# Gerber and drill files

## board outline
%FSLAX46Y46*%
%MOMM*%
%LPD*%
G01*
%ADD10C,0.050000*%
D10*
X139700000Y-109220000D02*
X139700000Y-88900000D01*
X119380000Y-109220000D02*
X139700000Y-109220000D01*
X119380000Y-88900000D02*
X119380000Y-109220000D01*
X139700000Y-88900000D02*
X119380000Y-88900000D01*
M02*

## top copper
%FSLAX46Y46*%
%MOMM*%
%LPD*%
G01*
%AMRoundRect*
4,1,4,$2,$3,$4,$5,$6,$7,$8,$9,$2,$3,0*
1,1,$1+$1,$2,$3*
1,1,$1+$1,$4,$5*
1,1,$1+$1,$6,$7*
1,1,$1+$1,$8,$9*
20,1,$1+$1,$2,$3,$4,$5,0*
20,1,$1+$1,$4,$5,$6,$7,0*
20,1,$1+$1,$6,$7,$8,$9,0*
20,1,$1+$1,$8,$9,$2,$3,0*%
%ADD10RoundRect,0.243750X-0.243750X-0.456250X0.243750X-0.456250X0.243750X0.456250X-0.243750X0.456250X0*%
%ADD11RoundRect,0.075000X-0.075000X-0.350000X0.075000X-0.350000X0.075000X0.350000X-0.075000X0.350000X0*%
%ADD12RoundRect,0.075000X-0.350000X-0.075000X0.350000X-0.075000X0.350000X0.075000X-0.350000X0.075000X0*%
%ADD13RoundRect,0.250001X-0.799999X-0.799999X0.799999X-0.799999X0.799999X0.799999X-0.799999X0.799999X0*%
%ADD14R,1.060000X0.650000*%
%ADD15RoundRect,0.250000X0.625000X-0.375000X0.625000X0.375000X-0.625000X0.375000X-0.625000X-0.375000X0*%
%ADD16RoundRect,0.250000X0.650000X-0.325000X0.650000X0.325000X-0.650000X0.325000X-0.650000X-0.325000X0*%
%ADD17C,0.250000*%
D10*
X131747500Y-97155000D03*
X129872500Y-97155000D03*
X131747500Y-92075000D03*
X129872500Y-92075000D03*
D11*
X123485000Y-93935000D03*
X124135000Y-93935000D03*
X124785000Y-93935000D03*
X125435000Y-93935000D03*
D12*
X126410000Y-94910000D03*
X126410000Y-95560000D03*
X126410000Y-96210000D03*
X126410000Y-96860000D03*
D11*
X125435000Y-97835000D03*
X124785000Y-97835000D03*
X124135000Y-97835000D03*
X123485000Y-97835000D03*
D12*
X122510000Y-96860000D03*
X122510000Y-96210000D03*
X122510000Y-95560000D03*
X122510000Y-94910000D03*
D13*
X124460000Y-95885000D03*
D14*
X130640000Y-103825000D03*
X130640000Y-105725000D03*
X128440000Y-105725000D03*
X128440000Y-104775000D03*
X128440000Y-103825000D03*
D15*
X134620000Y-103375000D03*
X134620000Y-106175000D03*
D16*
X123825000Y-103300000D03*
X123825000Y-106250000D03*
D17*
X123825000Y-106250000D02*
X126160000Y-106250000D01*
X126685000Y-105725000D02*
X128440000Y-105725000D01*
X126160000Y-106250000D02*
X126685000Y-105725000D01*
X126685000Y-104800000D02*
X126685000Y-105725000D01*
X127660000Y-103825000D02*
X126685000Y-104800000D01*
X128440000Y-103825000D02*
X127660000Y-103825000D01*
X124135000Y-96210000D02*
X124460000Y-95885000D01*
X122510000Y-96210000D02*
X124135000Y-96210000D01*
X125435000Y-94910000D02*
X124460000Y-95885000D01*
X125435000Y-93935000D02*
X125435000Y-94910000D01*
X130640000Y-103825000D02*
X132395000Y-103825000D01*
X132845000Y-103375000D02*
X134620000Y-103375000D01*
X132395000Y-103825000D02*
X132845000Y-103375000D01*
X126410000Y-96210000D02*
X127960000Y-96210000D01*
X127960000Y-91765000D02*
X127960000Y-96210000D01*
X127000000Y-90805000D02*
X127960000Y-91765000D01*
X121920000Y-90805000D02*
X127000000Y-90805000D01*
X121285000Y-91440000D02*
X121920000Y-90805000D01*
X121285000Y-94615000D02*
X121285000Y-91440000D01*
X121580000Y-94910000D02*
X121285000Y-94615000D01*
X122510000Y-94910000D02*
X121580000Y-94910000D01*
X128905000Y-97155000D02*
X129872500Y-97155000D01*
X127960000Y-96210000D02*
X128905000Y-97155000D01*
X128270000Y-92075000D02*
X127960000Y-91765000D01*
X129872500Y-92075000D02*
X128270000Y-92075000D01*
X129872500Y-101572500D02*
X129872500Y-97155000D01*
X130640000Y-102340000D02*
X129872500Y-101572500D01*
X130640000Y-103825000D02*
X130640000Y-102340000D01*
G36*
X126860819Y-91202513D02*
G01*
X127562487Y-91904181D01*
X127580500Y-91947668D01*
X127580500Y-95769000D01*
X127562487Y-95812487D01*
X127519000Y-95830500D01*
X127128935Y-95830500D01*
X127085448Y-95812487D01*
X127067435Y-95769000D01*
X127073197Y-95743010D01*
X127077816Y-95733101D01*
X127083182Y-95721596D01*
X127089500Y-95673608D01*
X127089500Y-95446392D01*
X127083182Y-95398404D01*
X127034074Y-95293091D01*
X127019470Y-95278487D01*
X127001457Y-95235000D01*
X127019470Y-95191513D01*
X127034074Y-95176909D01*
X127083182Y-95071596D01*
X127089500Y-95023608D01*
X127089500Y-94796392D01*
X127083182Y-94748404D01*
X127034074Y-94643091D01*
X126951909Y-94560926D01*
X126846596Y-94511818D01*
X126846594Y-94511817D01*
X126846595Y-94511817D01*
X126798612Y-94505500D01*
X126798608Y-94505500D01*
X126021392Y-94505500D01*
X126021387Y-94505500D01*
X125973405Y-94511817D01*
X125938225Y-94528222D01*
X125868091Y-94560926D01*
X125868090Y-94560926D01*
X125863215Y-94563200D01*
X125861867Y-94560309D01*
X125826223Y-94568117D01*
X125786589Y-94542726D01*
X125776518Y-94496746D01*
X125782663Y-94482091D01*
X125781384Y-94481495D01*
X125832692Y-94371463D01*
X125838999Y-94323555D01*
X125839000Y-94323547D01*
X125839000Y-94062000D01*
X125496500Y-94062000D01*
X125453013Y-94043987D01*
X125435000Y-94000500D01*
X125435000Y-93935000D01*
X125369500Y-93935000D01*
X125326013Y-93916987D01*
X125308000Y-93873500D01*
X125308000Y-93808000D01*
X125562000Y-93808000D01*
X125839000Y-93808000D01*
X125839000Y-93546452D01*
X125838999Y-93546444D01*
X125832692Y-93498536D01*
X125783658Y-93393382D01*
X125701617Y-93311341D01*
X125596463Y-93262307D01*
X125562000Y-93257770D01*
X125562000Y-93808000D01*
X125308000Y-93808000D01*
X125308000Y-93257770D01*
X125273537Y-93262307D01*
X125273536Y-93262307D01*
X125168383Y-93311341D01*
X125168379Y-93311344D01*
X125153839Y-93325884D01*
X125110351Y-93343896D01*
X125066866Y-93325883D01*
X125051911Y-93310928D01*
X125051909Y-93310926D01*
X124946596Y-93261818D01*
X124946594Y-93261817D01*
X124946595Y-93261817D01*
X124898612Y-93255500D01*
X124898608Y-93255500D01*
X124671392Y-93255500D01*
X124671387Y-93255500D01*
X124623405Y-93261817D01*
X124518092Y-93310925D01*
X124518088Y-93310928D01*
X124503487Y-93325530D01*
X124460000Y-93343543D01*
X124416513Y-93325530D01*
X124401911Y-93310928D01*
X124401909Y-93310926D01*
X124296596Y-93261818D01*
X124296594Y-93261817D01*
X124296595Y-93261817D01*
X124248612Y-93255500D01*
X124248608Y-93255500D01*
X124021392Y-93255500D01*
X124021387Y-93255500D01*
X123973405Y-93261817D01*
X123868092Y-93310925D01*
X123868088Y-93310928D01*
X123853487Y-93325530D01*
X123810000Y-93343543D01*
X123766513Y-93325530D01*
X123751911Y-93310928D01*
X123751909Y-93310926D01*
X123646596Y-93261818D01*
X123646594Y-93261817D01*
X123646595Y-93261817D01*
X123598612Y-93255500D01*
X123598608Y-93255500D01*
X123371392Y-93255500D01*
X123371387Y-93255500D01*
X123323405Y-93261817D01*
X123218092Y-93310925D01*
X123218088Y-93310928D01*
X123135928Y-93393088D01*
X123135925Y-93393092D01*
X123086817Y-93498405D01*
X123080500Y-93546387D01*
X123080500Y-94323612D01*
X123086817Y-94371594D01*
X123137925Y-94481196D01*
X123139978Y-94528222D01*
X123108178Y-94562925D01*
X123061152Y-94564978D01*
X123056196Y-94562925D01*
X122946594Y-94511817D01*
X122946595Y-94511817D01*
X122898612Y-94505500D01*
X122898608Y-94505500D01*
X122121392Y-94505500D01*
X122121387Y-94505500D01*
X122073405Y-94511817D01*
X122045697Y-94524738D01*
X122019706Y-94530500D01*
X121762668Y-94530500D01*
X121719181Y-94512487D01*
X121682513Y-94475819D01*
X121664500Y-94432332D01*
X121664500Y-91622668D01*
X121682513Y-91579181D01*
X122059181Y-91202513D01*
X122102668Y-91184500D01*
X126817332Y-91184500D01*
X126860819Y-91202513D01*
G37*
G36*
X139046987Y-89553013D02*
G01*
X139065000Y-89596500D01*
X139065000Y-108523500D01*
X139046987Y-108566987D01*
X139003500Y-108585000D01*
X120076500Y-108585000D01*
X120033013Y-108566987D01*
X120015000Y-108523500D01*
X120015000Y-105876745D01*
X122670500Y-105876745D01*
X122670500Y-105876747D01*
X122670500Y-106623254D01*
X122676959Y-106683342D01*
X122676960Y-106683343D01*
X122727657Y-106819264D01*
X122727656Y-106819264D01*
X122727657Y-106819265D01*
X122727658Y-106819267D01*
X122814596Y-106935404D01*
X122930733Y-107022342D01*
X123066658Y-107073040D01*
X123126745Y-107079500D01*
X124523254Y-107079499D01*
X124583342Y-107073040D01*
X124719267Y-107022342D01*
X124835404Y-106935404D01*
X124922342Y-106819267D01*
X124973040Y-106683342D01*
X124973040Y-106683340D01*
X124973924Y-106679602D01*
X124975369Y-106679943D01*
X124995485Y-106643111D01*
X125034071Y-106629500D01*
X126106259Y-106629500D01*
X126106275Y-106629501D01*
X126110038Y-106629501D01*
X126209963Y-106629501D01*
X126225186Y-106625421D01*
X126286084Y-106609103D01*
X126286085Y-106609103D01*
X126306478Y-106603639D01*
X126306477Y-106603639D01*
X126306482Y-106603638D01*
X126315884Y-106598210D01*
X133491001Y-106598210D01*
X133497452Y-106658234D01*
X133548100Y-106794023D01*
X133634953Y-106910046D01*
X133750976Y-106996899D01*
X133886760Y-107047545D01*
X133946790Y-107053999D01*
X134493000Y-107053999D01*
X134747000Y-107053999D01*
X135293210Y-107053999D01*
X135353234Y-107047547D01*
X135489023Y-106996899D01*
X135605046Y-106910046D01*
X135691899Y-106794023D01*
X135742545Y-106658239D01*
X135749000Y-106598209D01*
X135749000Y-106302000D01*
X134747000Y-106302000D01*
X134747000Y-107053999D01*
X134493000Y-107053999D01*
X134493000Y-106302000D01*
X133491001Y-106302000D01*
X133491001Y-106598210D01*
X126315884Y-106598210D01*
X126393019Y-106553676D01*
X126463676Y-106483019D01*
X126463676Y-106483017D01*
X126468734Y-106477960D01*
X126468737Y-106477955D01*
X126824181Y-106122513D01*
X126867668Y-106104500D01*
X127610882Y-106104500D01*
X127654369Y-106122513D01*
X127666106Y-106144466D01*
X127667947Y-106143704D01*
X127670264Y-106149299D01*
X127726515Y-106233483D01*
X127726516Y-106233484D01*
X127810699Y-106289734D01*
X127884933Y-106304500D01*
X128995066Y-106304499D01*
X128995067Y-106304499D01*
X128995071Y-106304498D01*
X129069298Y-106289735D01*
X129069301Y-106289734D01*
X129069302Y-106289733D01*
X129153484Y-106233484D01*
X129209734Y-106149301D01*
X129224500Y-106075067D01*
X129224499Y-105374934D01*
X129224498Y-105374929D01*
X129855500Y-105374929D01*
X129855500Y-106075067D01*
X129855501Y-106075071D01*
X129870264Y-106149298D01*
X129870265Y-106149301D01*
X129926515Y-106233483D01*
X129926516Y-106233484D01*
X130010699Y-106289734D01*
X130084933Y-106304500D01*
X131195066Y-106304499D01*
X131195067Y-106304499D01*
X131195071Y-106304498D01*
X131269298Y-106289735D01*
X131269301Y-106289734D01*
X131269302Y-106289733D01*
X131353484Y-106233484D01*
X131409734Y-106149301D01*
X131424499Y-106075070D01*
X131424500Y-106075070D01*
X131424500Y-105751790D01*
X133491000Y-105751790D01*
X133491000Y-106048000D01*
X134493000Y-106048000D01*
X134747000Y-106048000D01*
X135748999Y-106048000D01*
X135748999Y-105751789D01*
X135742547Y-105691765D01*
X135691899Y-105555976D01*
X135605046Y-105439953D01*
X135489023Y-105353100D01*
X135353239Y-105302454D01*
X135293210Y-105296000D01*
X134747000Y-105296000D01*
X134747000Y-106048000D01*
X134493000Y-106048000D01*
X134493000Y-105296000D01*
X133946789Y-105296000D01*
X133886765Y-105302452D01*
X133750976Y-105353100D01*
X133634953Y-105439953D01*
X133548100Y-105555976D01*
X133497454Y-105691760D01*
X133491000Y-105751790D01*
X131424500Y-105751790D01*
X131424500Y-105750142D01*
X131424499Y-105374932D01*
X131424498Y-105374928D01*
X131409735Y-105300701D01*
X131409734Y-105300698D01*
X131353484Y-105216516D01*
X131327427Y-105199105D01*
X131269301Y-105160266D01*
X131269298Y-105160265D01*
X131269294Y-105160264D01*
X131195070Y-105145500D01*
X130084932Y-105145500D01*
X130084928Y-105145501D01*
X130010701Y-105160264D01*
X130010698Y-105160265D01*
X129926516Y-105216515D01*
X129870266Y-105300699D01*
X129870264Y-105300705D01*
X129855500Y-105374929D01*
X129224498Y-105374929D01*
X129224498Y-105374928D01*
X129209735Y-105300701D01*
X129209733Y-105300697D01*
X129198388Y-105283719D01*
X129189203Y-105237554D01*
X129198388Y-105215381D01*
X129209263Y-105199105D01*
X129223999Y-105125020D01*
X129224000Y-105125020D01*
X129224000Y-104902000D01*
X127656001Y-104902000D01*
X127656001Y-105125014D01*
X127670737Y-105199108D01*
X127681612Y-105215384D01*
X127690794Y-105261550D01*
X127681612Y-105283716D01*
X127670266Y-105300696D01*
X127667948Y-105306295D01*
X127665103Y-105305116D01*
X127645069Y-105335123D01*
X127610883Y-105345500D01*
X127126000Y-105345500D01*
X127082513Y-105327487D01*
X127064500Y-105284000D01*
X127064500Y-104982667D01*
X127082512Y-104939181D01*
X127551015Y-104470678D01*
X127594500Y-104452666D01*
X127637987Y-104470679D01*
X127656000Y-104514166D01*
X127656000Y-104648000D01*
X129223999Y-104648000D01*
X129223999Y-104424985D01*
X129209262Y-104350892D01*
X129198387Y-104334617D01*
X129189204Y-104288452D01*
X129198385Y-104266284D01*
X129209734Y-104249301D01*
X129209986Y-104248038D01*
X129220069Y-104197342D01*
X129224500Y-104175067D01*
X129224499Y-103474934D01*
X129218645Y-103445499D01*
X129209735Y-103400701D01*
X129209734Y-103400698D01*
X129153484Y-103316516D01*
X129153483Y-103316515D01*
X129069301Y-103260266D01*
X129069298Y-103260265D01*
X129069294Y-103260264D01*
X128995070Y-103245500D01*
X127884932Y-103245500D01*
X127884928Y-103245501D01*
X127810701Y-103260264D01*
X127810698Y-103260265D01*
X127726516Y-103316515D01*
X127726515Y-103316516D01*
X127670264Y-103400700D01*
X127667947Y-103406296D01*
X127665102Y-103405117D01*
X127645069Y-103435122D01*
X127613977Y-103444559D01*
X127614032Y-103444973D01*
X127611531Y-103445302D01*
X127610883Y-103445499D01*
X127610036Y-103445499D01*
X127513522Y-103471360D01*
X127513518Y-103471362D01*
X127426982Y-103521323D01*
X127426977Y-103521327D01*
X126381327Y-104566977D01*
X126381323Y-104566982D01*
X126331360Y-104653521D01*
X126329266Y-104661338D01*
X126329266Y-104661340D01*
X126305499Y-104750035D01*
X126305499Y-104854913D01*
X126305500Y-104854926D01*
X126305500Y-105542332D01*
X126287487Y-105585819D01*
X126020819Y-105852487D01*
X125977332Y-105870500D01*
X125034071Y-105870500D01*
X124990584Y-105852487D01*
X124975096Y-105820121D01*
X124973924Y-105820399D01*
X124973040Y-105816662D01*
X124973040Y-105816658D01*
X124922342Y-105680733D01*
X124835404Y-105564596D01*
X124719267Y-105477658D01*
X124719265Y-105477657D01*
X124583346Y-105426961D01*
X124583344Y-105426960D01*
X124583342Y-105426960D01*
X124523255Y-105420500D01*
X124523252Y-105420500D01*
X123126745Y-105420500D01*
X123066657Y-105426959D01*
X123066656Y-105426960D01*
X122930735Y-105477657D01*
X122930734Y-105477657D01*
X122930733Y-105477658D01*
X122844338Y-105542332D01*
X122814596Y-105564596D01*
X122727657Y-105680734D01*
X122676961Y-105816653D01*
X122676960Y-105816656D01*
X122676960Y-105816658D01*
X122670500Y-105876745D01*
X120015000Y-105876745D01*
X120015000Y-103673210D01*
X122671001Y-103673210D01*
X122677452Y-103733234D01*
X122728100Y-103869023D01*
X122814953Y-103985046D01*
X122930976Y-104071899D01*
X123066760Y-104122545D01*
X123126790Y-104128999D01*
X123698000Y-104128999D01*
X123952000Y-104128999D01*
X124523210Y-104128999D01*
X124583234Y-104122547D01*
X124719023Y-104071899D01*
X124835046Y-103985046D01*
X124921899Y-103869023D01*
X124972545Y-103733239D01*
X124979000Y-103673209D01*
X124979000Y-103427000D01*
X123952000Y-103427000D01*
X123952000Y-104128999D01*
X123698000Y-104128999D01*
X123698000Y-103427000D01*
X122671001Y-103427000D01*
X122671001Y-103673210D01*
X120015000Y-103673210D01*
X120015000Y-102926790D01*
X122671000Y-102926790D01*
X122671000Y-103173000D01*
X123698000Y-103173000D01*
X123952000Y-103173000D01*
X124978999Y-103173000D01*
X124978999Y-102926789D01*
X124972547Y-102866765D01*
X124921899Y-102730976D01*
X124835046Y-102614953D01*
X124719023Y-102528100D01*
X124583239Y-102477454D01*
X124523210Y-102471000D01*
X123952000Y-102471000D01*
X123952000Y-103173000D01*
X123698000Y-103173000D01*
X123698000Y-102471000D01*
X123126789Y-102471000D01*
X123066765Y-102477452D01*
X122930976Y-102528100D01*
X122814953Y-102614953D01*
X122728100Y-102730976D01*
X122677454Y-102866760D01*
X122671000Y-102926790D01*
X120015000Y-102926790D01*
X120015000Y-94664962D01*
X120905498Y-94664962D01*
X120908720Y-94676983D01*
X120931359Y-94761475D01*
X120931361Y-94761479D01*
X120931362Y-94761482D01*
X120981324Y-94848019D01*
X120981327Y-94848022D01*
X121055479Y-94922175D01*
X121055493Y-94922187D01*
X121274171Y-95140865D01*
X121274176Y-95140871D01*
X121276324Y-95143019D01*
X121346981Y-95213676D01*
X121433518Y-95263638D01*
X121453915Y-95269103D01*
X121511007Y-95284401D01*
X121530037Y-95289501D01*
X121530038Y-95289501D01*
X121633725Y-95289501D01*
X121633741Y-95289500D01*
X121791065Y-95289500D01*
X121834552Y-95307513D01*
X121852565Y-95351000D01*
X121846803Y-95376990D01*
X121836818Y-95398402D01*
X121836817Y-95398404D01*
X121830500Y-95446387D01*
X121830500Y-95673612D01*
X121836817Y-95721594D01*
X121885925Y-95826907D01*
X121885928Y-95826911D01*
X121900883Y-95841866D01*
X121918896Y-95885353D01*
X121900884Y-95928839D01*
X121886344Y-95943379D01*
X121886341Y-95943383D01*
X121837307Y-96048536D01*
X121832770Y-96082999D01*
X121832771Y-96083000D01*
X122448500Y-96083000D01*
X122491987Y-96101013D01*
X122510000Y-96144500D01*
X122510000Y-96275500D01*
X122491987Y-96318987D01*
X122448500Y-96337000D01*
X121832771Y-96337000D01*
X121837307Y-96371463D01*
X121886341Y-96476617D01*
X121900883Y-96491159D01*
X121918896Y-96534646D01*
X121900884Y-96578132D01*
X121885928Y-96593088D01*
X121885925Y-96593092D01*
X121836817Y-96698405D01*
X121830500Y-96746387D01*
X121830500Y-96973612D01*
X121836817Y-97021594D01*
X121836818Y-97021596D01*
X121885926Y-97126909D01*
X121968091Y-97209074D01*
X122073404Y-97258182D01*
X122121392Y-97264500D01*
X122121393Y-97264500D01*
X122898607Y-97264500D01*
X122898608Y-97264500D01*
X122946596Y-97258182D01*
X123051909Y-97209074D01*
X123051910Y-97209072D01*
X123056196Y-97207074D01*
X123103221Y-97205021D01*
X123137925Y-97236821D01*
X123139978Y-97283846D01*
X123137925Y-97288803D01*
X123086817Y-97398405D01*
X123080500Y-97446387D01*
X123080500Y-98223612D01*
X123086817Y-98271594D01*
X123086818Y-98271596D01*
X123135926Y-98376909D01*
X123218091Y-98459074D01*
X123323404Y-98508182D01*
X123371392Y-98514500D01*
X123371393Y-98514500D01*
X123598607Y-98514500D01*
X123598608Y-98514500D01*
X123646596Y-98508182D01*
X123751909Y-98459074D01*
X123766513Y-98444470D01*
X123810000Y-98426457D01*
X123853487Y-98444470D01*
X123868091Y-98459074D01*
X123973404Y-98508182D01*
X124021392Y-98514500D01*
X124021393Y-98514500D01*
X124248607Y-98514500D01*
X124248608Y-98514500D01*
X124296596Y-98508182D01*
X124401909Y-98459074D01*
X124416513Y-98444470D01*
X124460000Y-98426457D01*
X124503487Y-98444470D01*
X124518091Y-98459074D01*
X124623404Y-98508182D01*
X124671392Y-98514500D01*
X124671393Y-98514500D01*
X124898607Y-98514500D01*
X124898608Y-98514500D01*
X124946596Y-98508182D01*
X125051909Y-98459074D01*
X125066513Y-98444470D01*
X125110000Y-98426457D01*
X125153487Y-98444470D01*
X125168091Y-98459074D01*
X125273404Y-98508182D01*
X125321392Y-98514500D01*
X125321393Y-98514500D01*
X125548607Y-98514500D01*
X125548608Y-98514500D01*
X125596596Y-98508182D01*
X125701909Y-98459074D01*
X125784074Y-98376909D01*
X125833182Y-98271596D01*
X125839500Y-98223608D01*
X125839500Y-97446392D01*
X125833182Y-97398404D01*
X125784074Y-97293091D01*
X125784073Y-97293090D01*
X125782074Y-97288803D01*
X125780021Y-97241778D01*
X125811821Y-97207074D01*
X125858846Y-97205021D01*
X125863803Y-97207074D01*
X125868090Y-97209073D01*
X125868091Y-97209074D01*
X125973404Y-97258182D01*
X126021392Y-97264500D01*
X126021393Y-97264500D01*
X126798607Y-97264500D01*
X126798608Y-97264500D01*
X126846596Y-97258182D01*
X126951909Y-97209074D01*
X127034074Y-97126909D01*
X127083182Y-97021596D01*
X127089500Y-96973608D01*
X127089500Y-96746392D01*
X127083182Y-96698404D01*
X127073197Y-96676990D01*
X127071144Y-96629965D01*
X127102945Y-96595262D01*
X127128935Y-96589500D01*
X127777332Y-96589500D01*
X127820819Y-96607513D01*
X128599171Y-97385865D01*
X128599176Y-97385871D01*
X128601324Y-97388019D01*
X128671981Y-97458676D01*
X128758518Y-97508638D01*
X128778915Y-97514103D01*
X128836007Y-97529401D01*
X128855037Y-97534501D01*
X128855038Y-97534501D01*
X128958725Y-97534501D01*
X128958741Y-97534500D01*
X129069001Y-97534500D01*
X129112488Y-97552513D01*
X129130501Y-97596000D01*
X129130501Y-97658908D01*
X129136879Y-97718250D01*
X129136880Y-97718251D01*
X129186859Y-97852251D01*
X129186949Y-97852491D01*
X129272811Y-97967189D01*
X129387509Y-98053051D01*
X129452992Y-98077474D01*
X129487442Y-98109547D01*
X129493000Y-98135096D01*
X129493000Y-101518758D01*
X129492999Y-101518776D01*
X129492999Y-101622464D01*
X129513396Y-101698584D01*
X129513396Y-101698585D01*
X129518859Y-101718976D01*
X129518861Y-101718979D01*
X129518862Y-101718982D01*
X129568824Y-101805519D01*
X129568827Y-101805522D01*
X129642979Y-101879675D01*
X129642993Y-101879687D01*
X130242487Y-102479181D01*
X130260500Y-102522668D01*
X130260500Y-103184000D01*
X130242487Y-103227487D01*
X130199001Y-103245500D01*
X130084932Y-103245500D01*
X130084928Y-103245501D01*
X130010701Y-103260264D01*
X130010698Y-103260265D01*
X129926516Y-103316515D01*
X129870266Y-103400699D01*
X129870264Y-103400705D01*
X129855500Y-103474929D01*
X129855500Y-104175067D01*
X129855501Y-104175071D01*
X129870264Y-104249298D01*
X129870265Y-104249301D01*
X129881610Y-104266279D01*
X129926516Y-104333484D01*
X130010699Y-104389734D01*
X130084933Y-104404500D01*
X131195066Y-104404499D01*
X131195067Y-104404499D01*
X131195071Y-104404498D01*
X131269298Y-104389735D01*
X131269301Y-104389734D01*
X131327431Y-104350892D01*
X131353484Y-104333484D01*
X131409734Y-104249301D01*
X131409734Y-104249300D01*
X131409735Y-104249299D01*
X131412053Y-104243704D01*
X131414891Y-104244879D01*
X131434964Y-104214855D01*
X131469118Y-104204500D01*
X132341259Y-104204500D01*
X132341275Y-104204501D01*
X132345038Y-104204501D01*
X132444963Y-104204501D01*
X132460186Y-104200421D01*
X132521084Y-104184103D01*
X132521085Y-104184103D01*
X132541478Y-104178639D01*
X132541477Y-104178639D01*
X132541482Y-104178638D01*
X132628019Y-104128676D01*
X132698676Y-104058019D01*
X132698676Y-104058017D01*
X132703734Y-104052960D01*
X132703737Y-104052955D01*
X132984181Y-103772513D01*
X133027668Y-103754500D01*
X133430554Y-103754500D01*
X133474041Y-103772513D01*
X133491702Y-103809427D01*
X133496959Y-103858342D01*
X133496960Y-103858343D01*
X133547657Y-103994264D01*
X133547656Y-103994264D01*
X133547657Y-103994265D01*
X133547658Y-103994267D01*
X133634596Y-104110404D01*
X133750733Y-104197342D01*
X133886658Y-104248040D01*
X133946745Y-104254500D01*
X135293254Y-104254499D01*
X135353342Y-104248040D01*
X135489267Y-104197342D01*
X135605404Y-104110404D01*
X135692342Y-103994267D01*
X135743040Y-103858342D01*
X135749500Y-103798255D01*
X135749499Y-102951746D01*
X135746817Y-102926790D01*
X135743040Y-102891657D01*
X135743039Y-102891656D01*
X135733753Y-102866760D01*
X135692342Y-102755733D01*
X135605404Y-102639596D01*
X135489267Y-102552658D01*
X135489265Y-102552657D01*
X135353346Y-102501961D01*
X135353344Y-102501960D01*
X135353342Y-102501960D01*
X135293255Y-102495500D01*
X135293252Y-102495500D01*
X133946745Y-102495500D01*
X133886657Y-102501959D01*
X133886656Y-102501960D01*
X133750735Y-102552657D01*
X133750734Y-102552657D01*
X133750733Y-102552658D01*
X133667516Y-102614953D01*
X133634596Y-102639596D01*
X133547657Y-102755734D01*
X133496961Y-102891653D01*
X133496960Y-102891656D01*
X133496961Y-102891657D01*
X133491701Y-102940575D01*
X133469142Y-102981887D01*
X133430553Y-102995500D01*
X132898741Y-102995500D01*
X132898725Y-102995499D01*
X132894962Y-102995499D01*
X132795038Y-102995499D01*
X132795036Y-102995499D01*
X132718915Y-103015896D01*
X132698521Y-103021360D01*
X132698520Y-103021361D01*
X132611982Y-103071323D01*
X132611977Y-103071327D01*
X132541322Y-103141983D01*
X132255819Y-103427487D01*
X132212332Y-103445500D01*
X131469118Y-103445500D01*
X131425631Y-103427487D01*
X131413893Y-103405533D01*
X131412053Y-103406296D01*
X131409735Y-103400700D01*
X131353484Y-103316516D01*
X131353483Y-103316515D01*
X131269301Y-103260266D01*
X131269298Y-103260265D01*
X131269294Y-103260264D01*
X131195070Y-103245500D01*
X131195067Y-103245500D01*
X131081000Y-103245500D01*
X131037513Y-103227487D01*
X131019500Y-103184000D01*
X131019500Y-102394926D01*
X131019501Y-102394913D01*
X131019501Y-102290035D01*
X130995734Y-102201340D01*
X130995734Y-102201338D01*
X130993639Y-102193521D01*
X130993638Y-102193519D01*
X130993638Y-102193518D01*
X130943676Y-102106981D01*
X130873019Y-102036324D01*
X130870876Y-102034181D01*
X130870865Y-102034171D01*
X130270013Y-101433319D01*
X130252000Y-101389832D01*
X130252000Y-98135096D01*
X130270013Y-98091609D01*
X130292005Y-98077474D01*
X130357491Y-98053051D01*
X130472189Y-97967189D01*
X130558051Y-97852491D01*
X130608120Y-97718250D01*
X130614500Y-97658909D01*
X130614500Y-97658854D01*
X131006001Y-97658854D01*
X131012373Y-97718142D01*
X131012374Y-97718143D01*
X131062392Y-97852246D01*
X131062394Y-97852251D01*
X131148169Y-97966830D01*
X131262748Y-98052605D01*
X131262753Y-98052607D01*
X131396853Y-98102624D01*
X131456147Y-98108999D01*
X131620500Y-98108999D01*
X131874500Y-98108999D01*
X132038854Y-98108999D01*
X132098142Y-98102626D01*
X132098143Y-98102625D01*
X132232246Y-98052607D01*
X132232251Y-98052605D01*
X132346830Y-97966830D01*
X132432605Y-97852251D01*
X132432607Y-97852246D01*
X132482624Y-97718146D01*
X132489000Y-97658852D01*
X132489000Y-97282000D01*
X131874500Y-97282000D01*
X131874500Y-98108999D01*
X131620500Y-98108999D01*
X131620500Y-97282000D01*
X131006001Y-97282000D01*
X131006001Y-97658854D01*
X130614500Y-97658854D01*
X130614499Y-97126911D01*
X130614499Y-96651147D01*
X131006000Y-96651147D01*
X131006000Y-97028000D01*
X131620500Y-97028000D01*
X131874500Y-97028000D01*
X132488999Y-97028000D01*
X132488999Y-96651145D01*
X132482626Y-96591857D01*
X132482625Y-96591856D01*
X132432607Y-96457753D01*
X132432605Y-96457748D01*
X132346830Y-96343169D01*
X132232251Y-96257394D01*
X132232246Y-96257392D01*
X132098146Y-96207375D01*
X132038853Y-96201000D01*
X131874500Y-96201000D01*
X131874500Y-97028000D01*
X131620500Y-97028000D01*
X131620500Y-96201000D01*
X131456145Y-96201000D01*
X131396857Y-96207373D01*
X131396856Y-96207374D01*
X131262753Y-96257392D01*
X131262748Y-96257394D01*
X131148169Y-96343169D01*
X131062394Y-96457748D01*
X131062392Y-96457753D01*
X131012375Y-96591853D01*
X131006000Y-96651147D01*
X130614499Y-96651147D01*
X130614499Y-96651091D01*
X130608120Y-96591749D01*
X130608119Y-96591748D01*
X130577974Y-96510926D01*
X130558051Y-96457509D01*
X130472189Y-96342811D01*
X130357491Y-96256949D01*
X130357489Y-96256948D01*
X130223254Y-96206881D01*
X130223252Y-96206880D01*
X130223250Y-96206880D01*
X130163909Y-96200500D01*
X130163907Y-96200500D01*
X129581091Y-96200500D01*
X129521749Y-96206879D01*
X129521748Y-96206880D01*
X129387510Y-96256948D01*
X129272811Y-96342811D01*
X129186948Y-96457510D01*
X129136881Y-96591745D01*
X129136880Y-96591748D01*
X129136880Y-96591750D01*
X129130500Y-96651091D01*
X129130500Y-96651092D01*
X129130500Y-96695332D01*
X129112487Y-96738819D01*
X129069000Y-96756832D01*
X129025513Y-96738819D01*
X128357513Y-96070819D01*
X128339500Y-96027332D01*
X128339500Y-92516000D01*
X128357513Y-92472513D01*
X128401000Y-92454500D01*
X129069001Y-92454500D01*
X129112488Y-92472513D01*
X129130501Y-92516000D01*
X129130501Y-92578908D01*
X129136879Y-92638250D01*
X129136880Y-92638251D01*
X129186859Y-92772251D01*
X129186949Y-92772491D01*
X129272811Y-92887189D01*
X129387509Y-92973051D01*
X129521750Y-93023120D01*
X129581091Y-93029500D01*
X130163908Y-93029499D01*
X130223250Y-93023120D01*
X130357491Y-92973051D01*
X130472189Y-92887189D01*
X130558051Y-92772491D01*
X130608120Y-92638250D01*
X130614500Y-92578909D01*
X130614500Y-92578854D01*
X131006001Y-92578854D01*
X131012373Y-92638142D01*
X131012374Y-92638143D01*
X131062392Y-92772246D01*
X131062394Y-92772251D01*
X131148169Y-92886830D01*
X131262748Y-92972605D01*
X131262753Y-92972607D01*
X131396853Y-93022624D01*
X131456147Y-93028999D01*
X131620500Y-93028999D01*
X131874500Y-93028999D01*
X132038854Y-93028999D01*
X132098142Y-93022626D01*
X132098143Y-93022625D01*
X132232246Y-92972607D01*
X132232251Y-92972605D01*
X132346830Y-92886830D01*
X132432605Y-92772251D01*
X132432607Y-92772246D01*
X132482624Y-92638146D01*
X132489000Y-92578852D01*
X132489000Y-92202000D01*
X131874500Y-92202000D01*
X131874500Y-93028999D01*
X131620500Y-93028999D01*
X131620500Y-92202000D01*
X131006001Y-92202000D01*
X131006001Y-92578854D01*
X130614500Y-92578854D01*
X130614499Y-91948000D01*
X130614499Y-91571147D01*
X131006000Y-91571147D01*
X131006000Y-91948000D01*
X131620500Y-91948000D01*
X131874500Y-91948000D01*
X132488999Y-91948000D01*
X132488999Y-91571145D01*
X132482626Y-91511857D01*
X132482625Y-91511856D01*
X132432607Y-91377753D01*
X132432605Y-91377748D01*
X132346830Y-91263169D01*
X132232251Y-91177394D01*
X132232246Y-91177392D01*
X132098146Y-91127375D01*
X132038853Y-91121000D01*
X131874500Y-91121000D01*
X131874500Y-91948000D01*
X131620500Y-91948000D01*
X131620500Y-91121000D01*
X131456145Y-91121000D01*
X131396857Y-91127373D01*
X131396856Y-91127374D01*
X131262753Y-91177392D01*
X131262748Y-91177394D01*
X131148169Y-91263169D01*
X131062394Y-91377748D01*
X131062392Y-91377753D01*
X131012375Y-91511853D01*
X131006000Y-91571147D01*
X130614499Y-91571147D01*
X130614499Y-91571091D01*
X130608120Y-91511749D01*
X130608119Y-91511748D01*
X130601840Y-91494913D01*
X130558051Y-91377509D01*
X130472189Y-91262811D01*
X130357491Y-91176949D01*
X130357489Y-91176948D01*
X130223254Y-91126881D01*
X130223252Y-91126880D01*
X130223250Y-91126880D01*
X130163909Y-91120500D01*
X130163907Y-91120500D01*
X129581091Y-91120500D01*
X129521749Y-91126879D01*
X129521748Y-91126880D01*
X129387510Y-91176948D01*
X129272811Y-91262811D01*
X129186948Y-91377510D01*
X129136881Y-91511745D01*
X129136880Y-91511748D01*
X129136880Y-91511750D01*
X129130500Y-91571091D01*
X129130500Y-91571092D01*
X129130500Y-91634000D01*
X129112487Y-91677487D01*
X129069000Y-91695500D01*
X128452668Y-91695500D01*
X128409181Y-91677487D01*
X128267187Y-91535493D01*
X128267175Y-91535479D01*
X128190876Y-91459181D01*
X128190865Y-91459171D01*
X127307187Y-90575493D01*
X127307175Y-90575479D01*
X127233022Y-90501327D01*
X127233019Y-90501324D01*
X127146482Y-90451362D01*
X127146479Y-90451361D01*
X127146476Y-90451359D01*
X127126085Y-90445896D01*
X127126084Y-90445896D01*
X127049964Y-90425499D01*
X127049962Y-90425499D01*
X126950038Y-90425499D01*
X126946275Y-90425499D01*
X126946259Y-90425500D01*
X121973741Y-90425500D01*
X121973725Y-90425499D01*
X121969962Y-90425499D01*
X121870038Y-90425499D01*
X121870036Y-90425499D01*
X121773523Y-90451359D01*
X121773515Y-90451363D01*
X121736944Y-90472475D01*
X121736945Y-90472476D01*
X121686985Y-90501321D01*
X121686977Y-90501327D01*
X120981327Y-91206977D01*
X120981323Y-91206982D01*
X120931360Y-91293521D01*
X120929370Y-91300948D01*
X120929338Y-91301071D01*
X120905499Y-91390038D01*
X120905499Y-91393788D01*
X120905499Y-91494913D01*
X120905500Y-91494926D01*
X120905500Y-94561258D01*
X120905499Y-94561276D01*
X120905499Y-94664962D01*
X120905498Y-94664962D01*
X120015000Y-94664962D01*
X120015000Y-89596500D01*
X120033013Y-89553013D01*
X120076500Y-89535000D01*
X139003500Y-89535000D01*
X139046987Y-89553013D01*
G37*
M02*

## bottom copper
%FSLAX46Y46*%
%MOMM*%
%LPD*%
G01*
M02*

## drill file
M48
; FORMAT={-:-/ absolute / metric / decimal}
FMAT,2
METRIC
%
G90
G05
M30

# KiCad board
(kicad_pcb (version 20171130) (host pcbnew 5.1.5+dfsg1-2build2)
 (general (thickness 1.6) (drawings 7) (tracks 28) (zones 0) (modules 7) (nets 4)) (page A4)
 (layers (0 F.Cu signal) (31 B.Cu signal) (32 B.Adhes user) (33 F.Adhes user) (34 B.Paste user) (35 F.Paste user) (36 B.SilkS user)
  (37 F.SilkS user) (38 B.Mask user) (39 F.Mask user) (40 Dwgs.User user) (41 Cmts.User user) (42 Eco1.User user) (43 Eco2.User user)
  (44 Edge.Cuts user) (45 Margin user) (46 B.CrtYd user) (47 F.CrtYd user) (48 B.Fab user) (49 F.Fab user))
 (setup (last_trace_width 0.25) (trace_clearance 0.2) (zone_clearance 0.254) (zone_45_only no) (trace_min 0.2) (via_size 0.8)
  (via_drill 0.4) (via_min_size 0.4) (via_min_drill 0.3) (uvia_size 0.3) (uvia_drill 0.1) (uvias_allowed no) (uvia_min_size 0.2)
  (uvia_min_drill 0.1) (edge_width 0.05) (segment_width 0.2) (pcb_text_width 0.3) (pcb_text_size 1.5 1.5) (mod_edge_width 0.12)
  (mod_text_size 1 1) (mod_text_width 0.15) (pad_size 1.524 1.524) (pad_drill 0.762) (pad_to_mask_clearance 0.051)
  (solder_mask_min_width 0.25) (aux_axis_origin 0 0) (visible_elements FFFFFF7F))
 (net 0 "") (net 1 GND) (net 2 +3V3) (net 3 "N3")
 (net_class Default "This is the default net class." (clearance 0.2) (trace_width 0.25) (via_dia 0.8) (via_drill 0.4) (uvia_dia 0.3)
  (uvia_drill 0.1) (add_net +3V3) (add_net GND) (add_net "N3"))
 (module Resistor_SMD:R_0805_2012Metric (layer F.Cu) (at 130.81 97.155)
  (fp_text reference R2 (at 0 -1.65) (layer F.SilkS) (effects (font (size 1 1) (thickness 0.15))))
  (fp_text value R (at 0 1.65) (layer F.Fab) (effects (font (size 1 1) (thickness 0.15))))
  (pad 2 smd roundrect (at 0.9375 0) (size 0.975 1.4) (layers F.Cu F.Paste F.Mask) (roundrect_rratio 0.25) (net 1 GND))
  (pad 1 smd roundrect (at -0.9375 0) (size 0.975 1.4) (layers F.Cu F.Paste F.Mask) (roundrect_rratio 0.25) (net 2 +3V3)))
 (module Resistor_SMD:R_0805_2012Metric (layer F.Cu) (at 130.81 92.075)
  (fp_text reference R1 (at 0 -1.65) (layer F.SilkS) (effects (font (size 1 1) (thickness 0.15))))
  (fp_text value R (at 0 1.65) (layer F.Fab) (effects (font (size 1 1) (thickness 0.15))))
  (pad 2 smd roundrect (at 0.9375 0) (size 0.975 1.4) (layers F.Cu F.Paste F.Mask) (roundrect_rratio 0.25) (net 1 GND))
  (pad 1 smd roundrect (at -0.9375 0) (size 0.975 1.4) (layers F.Cu F.Paste F.Mask) (roundrect_rratio 0.25) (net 2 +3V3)))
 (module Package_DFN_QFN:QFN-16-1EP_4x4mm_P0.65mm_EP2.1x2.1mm (layer F.Cu) (at 124.46 95.885)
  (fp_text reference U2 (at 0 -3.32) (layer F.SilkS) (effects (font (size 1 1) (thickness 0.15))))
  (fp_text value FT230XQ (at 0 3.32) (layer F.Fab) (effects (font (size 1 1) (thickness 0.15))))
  (pad 16 smd roundrect (at -0.975 -1.95) (size 0.3 0.85) (layers F.Cu F.Paste F.Mask) (roundrect_rratio 0.25))
  (pad 15 smd roundrect (at -0.325 -1.95) (size 0.3 0.85) (layers F.Cu F.Paste F.Mask) (roundrect_rratio 0.25))
  (pad 14 smd roundrect (at 0.325 -1.95) (size 0.3 0.85) (layers F.Cu F.Paste F.Mask) (roundrect_rratio 0.25))
  (pad 13 smd roundrect (at 0.975 -1.95) (size 0.3 0.85) (layers F.Cu F.Paste F.Mask) (roundrect_rratio 0.25) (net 1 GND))
  (pad 12 smd roundrect (at 1.95 -0.975) (size 0.85 0.3) (layers F.Cu F.Paste F.Mask) (roundrect_rratio 0.25))
  (pad 11 smd roundrect (at 1.95 -0.325) (size 0.85 0.3) (layers F.Cu F.Paste F.Mask) (roundrect_rratio 0.25))
  (pad 10 smd roundrect (at 1.95 0.325) (size 0.85 0.3) (layers F.Cu F.Paste F.Mask) (roundrect_rratio 0.25) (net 2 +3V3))
  (pad 9 smd roundrect (at 1.95 0.975) (size 0.85 0.3) (layers F.Cu F.Paste F.Mask) (roundrect_rratio 0.25))
  (pad 8 smd roundrect (at 0.975 1.95) (size 0.3 0.85) (layers F.Cu F.Paste F.Mask) (roundrect_rratio 0.25))
  (pad 7 smd roundrect (at 0.325 1.95) (size 0.3 0.85) (layers F.Cu F.Paste F.Mask) (roundrect_rratio 0.25))
  (pad 6 smd roundrect (at -0.325 1.95) (size 0.3 0.85) (layers F.Cu F.Paste F.Mask) (roundrect_rratio 0.25))
  (pad 5 smd roundrect (at -0.975 1.95) (size 0.3 0.85) (layers F.Cu F.Paste F.Mask) (roundrect_rratio 0.25))
  (pad 4 smd roundrect (at -1.95 0.975) (size 0.85 0.3) (layers F.Cu F.Paste F.Mask) (roundrect_rratio 0.25))
  (pad 3 smd roundrect (at -1.95 0.325) (size 0.85 0.3) (layers F.Cu F.Paste F.Mask) (roundrect_rratio 0.25) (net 1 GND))
  (pad 2 smd roundrect (at -1.95 -0.325) (size 0.85 0.3) (layers F.Cu F.Paste F.Mask) (roundrect_rratio 0.25))
  (pad 1 smd roundrect (at -1.95 -0.975) (size 0.85 0.3) (layers F.Cu F.Paste F.Mask) (roundrect_rratio 0.25) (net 2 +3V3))
  (pad "" smd roundrect (at 0.525 0.525) (size 0.85 0.85) (layers F.Paste) (roundrect_rratio 0.25))
  (pad "" smd roundrect (at 0.525 -0.525) (size 0.85 0.85) (layers F.Paste) (roundrect_rratio 0.25))
  (pad "" smd roundrect (at -0.525 0.525) (size 0.85 0.85) (layers F.Paste) (roundrect_rratio 0.25))
  (pad "" smd roundrect (at -0.525 -0.525) (size 0.85 0.85) (layers F.Paste) (roundrect_rratio 0.25))
  (pad 17 smd roundrect (at 0 0) (size 2.1 2.1) (layers F.Cu F.Mask) (roundrect_rratio 0.119048) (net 1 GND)))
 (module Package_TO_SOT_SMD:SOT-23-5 (layer F.Cu) (at 129.54 104.775)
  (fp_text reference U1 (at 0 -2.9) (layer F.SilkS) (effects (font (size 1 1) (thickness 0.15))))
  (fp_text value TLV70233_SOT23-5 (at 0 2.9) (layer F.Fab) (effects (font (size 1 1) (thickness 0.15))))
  (pad 5 smd rect (at 1.1 -0.95) (size 1.06 0.65) (layers F.Cu F.Paste F.Mask) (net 2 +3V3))
  (pad 4 smd rect (at 1.1 0.95) (size 1.06 0.65) (layers F.Cu F.Paste F.Mask))
  (pad 3 smd rect (at -1.1 0.95) (size 1.06 0.65) (layers F.Cu F.Paste F.Mask) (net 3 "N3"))
  (pad 2 smd rect (at -1.1 0) (size 1.06 0.65) (layers F.Cu F.Paste F.Mask) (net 1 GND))
  (pad 1 smd rect (at -1.1 -0.95) (size 1.06 0.65) (layers F.Cu F.Paste F.Mask) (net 3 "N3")))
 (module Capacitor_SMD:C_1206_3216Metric (layer F.Cu) (at 134.62 104.775 90)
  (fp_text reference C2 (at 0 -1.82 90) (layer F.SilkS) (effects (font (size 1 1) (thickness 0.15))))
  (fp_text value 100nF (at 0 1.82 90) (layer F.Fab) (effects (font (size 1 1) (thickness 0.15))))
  (pad 2 smd roundrect (at 1.4 0 90) (size 1.25 1.75) (layers F.Cu F.Paste F.Mask) (roundrect_rratio 0.2) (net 2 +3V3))
  (pad 1 smd roundrect (at -1.4 0 90) (size 1.25 1.75) (layers F.Cu F.Paste F.Mask) (roundrect_rratio 0.2) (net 1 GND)))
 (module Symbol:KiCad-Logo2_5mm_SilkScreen (layer F.Cu) (at 135.89 95.885 90)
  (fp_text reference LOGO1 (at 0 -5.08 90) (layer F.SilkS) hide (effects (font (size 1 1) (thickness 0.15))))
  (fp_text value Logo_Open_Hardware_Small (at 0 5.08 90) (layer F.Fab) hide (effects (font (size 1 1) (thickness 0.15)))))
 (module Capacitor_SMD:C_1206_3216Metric (layer F.Cu) (at 123.825 104.775 90)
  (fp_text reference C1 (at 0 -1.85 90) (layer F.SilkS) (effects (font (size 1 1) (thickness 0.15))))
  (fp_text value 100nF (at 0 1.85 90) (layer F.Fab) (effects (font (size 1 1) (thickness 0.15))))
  (pad 2 smd roundrect (at 1.475 0 90) (size 1.15 1.8) (layers F.Cu F.Paste F.Mask) (roundrect_rratio 0.217391) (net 1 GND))
  (pad 1 smd roundrect (at -1.475 0 90) (size 1.15 1.8) (layers F.Cu F.Paste F.Mask) (roundrect_rratio 0.217391) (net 3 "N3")))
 (gr_line (start 139.7 109.22) (end 139.7 88.9) (layer Edge.Cuts) (width 0.05))
 (gr_line (start 119.38 109.22) (end 139.7 109.22) (layer Edge.Cuts) (width 0.05))
 (gr_line (start 119.38 88.9) (end 119.38 109.22) (layer Edge.Cuts) (width 0.05))
 (gr_line (start 139.7 88.9) (end 119.38 88.9) (layer Edge.Cuts) (width 0.05))
 (segment (start 123.825 106.25) (end 126.16 106.25) (width 0.25) (layer F.Cu) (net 3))
 (segment (start 126.685 105.725) (end 128.44 105.725) (width 0.25) (layer F.Cu) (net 3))
 (segment (start 126.16 106.25) (end 126.685 105.725) (width 0.25) (layer F.Cu) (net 3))
 (segment (start 126.685 104.8) (end 126.685 105.725) (width 0.25) (layer F.Cu) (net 3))
 (segment (start 127.66 103.825) (end 126.685 104.8) (width 0.25) (layer F.Cu) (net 3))
 (segment (start 128.44 103.825) (end 127.66 103.825) (width 0.25) (layer F.Cu) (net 3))
 (segment (start 124.135 96.21) (end 124.46 95.885) (width 0.25) (layer F.Cu) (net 1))
 (segment (start 122.51 96.21) (end 124.135 96.21) (width 0.25) (layer F.Cu) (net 1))
 (segment (start 125.435 94.91) (end 124.46 95.885) (width 0.25) (layer F.Cu) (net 1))
 (segment (start 125.435 93.935) (end 125.435 94.91) (width 0.25) (layer F.Cu) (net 1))
 (segment (start 130.64 103.825) (end 132.395 103.825) (width 0.25) (layer F.Cu) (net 2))
 (segment (start 132.845 103.375) (end 134.62 103.375) (width 0.25) (layer F.Cu) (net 2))
 (segment (start 132.395 103.825) (end 132.845 103.375) (width 0.25) (layer F.Cu) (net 2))
 (segment (start 126.41 96.21) (end 127.96 96.21) (width 0.25) (layer F.Cu) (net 2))
 (segment (start 127.96 91.765) (end 127.96 96.21) (width 0.25) (layer F.Cu) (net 2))
 (segment (start 127 90.805) (end 127.96 91.765) (width 0.25) (layer F.Cu) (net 2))
 (segment (start 121.92 90.805) (end 127 90.805) (width 0.25) (layer F.Cu) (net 2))
 (segment (start 121.285 91.44) (end 121.92 90.805) (width 0.25) (layer F.Cu) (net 2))
 (segment (start 121.285 94.615) (end 121.285 91.44) (width 0.25) (layer F.Cu) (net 2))
 (segment (start 121.58 94.91) (end 121.285 94.615) (width 0.25) (layer F.Cu) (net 2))
 (segment (start 122.51 94.91) (end 121.58 94.91) (width 0.25) (layer F.Cu) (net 2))
 (segment (start 128.905 97.155) (end 129.8725 97.155) (width 0.25) (layer F.Cu) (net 2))
 (segment (start 127.96 96.21) (end 128.905 97.155) (width 0.25) (layer F.Cu) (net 2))
 (segment (start 128.27 92.075) (end 127.96 91.765) (width 0.25) (layer F.Cu) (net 2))
 (segment (start 129.8725 92.075) (end 128.27 92.075) (width 0.25) (layer F.Cu) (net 2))
 (segment (start 129.8725 101.5725) (end 129.8725 97.155) (width 0.25) (layer F.Cu) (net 2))
 (segment (start 130.64 102.34) (end 129.8725 101.5725) (width 0.25) (layer F.Cu) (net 2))
 (segment (start 130.64 103.825) (end 130.64 102.34) (width 0.25) (layer F.Cu) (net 2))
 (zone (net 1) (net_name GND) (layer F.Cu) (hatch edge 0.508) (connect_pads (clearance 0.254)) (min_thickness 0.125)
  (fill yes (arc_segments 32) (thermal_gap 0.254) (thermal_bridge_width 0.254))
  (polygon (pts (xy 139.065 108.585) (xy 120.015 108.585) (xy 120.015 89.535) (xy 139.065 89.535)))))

